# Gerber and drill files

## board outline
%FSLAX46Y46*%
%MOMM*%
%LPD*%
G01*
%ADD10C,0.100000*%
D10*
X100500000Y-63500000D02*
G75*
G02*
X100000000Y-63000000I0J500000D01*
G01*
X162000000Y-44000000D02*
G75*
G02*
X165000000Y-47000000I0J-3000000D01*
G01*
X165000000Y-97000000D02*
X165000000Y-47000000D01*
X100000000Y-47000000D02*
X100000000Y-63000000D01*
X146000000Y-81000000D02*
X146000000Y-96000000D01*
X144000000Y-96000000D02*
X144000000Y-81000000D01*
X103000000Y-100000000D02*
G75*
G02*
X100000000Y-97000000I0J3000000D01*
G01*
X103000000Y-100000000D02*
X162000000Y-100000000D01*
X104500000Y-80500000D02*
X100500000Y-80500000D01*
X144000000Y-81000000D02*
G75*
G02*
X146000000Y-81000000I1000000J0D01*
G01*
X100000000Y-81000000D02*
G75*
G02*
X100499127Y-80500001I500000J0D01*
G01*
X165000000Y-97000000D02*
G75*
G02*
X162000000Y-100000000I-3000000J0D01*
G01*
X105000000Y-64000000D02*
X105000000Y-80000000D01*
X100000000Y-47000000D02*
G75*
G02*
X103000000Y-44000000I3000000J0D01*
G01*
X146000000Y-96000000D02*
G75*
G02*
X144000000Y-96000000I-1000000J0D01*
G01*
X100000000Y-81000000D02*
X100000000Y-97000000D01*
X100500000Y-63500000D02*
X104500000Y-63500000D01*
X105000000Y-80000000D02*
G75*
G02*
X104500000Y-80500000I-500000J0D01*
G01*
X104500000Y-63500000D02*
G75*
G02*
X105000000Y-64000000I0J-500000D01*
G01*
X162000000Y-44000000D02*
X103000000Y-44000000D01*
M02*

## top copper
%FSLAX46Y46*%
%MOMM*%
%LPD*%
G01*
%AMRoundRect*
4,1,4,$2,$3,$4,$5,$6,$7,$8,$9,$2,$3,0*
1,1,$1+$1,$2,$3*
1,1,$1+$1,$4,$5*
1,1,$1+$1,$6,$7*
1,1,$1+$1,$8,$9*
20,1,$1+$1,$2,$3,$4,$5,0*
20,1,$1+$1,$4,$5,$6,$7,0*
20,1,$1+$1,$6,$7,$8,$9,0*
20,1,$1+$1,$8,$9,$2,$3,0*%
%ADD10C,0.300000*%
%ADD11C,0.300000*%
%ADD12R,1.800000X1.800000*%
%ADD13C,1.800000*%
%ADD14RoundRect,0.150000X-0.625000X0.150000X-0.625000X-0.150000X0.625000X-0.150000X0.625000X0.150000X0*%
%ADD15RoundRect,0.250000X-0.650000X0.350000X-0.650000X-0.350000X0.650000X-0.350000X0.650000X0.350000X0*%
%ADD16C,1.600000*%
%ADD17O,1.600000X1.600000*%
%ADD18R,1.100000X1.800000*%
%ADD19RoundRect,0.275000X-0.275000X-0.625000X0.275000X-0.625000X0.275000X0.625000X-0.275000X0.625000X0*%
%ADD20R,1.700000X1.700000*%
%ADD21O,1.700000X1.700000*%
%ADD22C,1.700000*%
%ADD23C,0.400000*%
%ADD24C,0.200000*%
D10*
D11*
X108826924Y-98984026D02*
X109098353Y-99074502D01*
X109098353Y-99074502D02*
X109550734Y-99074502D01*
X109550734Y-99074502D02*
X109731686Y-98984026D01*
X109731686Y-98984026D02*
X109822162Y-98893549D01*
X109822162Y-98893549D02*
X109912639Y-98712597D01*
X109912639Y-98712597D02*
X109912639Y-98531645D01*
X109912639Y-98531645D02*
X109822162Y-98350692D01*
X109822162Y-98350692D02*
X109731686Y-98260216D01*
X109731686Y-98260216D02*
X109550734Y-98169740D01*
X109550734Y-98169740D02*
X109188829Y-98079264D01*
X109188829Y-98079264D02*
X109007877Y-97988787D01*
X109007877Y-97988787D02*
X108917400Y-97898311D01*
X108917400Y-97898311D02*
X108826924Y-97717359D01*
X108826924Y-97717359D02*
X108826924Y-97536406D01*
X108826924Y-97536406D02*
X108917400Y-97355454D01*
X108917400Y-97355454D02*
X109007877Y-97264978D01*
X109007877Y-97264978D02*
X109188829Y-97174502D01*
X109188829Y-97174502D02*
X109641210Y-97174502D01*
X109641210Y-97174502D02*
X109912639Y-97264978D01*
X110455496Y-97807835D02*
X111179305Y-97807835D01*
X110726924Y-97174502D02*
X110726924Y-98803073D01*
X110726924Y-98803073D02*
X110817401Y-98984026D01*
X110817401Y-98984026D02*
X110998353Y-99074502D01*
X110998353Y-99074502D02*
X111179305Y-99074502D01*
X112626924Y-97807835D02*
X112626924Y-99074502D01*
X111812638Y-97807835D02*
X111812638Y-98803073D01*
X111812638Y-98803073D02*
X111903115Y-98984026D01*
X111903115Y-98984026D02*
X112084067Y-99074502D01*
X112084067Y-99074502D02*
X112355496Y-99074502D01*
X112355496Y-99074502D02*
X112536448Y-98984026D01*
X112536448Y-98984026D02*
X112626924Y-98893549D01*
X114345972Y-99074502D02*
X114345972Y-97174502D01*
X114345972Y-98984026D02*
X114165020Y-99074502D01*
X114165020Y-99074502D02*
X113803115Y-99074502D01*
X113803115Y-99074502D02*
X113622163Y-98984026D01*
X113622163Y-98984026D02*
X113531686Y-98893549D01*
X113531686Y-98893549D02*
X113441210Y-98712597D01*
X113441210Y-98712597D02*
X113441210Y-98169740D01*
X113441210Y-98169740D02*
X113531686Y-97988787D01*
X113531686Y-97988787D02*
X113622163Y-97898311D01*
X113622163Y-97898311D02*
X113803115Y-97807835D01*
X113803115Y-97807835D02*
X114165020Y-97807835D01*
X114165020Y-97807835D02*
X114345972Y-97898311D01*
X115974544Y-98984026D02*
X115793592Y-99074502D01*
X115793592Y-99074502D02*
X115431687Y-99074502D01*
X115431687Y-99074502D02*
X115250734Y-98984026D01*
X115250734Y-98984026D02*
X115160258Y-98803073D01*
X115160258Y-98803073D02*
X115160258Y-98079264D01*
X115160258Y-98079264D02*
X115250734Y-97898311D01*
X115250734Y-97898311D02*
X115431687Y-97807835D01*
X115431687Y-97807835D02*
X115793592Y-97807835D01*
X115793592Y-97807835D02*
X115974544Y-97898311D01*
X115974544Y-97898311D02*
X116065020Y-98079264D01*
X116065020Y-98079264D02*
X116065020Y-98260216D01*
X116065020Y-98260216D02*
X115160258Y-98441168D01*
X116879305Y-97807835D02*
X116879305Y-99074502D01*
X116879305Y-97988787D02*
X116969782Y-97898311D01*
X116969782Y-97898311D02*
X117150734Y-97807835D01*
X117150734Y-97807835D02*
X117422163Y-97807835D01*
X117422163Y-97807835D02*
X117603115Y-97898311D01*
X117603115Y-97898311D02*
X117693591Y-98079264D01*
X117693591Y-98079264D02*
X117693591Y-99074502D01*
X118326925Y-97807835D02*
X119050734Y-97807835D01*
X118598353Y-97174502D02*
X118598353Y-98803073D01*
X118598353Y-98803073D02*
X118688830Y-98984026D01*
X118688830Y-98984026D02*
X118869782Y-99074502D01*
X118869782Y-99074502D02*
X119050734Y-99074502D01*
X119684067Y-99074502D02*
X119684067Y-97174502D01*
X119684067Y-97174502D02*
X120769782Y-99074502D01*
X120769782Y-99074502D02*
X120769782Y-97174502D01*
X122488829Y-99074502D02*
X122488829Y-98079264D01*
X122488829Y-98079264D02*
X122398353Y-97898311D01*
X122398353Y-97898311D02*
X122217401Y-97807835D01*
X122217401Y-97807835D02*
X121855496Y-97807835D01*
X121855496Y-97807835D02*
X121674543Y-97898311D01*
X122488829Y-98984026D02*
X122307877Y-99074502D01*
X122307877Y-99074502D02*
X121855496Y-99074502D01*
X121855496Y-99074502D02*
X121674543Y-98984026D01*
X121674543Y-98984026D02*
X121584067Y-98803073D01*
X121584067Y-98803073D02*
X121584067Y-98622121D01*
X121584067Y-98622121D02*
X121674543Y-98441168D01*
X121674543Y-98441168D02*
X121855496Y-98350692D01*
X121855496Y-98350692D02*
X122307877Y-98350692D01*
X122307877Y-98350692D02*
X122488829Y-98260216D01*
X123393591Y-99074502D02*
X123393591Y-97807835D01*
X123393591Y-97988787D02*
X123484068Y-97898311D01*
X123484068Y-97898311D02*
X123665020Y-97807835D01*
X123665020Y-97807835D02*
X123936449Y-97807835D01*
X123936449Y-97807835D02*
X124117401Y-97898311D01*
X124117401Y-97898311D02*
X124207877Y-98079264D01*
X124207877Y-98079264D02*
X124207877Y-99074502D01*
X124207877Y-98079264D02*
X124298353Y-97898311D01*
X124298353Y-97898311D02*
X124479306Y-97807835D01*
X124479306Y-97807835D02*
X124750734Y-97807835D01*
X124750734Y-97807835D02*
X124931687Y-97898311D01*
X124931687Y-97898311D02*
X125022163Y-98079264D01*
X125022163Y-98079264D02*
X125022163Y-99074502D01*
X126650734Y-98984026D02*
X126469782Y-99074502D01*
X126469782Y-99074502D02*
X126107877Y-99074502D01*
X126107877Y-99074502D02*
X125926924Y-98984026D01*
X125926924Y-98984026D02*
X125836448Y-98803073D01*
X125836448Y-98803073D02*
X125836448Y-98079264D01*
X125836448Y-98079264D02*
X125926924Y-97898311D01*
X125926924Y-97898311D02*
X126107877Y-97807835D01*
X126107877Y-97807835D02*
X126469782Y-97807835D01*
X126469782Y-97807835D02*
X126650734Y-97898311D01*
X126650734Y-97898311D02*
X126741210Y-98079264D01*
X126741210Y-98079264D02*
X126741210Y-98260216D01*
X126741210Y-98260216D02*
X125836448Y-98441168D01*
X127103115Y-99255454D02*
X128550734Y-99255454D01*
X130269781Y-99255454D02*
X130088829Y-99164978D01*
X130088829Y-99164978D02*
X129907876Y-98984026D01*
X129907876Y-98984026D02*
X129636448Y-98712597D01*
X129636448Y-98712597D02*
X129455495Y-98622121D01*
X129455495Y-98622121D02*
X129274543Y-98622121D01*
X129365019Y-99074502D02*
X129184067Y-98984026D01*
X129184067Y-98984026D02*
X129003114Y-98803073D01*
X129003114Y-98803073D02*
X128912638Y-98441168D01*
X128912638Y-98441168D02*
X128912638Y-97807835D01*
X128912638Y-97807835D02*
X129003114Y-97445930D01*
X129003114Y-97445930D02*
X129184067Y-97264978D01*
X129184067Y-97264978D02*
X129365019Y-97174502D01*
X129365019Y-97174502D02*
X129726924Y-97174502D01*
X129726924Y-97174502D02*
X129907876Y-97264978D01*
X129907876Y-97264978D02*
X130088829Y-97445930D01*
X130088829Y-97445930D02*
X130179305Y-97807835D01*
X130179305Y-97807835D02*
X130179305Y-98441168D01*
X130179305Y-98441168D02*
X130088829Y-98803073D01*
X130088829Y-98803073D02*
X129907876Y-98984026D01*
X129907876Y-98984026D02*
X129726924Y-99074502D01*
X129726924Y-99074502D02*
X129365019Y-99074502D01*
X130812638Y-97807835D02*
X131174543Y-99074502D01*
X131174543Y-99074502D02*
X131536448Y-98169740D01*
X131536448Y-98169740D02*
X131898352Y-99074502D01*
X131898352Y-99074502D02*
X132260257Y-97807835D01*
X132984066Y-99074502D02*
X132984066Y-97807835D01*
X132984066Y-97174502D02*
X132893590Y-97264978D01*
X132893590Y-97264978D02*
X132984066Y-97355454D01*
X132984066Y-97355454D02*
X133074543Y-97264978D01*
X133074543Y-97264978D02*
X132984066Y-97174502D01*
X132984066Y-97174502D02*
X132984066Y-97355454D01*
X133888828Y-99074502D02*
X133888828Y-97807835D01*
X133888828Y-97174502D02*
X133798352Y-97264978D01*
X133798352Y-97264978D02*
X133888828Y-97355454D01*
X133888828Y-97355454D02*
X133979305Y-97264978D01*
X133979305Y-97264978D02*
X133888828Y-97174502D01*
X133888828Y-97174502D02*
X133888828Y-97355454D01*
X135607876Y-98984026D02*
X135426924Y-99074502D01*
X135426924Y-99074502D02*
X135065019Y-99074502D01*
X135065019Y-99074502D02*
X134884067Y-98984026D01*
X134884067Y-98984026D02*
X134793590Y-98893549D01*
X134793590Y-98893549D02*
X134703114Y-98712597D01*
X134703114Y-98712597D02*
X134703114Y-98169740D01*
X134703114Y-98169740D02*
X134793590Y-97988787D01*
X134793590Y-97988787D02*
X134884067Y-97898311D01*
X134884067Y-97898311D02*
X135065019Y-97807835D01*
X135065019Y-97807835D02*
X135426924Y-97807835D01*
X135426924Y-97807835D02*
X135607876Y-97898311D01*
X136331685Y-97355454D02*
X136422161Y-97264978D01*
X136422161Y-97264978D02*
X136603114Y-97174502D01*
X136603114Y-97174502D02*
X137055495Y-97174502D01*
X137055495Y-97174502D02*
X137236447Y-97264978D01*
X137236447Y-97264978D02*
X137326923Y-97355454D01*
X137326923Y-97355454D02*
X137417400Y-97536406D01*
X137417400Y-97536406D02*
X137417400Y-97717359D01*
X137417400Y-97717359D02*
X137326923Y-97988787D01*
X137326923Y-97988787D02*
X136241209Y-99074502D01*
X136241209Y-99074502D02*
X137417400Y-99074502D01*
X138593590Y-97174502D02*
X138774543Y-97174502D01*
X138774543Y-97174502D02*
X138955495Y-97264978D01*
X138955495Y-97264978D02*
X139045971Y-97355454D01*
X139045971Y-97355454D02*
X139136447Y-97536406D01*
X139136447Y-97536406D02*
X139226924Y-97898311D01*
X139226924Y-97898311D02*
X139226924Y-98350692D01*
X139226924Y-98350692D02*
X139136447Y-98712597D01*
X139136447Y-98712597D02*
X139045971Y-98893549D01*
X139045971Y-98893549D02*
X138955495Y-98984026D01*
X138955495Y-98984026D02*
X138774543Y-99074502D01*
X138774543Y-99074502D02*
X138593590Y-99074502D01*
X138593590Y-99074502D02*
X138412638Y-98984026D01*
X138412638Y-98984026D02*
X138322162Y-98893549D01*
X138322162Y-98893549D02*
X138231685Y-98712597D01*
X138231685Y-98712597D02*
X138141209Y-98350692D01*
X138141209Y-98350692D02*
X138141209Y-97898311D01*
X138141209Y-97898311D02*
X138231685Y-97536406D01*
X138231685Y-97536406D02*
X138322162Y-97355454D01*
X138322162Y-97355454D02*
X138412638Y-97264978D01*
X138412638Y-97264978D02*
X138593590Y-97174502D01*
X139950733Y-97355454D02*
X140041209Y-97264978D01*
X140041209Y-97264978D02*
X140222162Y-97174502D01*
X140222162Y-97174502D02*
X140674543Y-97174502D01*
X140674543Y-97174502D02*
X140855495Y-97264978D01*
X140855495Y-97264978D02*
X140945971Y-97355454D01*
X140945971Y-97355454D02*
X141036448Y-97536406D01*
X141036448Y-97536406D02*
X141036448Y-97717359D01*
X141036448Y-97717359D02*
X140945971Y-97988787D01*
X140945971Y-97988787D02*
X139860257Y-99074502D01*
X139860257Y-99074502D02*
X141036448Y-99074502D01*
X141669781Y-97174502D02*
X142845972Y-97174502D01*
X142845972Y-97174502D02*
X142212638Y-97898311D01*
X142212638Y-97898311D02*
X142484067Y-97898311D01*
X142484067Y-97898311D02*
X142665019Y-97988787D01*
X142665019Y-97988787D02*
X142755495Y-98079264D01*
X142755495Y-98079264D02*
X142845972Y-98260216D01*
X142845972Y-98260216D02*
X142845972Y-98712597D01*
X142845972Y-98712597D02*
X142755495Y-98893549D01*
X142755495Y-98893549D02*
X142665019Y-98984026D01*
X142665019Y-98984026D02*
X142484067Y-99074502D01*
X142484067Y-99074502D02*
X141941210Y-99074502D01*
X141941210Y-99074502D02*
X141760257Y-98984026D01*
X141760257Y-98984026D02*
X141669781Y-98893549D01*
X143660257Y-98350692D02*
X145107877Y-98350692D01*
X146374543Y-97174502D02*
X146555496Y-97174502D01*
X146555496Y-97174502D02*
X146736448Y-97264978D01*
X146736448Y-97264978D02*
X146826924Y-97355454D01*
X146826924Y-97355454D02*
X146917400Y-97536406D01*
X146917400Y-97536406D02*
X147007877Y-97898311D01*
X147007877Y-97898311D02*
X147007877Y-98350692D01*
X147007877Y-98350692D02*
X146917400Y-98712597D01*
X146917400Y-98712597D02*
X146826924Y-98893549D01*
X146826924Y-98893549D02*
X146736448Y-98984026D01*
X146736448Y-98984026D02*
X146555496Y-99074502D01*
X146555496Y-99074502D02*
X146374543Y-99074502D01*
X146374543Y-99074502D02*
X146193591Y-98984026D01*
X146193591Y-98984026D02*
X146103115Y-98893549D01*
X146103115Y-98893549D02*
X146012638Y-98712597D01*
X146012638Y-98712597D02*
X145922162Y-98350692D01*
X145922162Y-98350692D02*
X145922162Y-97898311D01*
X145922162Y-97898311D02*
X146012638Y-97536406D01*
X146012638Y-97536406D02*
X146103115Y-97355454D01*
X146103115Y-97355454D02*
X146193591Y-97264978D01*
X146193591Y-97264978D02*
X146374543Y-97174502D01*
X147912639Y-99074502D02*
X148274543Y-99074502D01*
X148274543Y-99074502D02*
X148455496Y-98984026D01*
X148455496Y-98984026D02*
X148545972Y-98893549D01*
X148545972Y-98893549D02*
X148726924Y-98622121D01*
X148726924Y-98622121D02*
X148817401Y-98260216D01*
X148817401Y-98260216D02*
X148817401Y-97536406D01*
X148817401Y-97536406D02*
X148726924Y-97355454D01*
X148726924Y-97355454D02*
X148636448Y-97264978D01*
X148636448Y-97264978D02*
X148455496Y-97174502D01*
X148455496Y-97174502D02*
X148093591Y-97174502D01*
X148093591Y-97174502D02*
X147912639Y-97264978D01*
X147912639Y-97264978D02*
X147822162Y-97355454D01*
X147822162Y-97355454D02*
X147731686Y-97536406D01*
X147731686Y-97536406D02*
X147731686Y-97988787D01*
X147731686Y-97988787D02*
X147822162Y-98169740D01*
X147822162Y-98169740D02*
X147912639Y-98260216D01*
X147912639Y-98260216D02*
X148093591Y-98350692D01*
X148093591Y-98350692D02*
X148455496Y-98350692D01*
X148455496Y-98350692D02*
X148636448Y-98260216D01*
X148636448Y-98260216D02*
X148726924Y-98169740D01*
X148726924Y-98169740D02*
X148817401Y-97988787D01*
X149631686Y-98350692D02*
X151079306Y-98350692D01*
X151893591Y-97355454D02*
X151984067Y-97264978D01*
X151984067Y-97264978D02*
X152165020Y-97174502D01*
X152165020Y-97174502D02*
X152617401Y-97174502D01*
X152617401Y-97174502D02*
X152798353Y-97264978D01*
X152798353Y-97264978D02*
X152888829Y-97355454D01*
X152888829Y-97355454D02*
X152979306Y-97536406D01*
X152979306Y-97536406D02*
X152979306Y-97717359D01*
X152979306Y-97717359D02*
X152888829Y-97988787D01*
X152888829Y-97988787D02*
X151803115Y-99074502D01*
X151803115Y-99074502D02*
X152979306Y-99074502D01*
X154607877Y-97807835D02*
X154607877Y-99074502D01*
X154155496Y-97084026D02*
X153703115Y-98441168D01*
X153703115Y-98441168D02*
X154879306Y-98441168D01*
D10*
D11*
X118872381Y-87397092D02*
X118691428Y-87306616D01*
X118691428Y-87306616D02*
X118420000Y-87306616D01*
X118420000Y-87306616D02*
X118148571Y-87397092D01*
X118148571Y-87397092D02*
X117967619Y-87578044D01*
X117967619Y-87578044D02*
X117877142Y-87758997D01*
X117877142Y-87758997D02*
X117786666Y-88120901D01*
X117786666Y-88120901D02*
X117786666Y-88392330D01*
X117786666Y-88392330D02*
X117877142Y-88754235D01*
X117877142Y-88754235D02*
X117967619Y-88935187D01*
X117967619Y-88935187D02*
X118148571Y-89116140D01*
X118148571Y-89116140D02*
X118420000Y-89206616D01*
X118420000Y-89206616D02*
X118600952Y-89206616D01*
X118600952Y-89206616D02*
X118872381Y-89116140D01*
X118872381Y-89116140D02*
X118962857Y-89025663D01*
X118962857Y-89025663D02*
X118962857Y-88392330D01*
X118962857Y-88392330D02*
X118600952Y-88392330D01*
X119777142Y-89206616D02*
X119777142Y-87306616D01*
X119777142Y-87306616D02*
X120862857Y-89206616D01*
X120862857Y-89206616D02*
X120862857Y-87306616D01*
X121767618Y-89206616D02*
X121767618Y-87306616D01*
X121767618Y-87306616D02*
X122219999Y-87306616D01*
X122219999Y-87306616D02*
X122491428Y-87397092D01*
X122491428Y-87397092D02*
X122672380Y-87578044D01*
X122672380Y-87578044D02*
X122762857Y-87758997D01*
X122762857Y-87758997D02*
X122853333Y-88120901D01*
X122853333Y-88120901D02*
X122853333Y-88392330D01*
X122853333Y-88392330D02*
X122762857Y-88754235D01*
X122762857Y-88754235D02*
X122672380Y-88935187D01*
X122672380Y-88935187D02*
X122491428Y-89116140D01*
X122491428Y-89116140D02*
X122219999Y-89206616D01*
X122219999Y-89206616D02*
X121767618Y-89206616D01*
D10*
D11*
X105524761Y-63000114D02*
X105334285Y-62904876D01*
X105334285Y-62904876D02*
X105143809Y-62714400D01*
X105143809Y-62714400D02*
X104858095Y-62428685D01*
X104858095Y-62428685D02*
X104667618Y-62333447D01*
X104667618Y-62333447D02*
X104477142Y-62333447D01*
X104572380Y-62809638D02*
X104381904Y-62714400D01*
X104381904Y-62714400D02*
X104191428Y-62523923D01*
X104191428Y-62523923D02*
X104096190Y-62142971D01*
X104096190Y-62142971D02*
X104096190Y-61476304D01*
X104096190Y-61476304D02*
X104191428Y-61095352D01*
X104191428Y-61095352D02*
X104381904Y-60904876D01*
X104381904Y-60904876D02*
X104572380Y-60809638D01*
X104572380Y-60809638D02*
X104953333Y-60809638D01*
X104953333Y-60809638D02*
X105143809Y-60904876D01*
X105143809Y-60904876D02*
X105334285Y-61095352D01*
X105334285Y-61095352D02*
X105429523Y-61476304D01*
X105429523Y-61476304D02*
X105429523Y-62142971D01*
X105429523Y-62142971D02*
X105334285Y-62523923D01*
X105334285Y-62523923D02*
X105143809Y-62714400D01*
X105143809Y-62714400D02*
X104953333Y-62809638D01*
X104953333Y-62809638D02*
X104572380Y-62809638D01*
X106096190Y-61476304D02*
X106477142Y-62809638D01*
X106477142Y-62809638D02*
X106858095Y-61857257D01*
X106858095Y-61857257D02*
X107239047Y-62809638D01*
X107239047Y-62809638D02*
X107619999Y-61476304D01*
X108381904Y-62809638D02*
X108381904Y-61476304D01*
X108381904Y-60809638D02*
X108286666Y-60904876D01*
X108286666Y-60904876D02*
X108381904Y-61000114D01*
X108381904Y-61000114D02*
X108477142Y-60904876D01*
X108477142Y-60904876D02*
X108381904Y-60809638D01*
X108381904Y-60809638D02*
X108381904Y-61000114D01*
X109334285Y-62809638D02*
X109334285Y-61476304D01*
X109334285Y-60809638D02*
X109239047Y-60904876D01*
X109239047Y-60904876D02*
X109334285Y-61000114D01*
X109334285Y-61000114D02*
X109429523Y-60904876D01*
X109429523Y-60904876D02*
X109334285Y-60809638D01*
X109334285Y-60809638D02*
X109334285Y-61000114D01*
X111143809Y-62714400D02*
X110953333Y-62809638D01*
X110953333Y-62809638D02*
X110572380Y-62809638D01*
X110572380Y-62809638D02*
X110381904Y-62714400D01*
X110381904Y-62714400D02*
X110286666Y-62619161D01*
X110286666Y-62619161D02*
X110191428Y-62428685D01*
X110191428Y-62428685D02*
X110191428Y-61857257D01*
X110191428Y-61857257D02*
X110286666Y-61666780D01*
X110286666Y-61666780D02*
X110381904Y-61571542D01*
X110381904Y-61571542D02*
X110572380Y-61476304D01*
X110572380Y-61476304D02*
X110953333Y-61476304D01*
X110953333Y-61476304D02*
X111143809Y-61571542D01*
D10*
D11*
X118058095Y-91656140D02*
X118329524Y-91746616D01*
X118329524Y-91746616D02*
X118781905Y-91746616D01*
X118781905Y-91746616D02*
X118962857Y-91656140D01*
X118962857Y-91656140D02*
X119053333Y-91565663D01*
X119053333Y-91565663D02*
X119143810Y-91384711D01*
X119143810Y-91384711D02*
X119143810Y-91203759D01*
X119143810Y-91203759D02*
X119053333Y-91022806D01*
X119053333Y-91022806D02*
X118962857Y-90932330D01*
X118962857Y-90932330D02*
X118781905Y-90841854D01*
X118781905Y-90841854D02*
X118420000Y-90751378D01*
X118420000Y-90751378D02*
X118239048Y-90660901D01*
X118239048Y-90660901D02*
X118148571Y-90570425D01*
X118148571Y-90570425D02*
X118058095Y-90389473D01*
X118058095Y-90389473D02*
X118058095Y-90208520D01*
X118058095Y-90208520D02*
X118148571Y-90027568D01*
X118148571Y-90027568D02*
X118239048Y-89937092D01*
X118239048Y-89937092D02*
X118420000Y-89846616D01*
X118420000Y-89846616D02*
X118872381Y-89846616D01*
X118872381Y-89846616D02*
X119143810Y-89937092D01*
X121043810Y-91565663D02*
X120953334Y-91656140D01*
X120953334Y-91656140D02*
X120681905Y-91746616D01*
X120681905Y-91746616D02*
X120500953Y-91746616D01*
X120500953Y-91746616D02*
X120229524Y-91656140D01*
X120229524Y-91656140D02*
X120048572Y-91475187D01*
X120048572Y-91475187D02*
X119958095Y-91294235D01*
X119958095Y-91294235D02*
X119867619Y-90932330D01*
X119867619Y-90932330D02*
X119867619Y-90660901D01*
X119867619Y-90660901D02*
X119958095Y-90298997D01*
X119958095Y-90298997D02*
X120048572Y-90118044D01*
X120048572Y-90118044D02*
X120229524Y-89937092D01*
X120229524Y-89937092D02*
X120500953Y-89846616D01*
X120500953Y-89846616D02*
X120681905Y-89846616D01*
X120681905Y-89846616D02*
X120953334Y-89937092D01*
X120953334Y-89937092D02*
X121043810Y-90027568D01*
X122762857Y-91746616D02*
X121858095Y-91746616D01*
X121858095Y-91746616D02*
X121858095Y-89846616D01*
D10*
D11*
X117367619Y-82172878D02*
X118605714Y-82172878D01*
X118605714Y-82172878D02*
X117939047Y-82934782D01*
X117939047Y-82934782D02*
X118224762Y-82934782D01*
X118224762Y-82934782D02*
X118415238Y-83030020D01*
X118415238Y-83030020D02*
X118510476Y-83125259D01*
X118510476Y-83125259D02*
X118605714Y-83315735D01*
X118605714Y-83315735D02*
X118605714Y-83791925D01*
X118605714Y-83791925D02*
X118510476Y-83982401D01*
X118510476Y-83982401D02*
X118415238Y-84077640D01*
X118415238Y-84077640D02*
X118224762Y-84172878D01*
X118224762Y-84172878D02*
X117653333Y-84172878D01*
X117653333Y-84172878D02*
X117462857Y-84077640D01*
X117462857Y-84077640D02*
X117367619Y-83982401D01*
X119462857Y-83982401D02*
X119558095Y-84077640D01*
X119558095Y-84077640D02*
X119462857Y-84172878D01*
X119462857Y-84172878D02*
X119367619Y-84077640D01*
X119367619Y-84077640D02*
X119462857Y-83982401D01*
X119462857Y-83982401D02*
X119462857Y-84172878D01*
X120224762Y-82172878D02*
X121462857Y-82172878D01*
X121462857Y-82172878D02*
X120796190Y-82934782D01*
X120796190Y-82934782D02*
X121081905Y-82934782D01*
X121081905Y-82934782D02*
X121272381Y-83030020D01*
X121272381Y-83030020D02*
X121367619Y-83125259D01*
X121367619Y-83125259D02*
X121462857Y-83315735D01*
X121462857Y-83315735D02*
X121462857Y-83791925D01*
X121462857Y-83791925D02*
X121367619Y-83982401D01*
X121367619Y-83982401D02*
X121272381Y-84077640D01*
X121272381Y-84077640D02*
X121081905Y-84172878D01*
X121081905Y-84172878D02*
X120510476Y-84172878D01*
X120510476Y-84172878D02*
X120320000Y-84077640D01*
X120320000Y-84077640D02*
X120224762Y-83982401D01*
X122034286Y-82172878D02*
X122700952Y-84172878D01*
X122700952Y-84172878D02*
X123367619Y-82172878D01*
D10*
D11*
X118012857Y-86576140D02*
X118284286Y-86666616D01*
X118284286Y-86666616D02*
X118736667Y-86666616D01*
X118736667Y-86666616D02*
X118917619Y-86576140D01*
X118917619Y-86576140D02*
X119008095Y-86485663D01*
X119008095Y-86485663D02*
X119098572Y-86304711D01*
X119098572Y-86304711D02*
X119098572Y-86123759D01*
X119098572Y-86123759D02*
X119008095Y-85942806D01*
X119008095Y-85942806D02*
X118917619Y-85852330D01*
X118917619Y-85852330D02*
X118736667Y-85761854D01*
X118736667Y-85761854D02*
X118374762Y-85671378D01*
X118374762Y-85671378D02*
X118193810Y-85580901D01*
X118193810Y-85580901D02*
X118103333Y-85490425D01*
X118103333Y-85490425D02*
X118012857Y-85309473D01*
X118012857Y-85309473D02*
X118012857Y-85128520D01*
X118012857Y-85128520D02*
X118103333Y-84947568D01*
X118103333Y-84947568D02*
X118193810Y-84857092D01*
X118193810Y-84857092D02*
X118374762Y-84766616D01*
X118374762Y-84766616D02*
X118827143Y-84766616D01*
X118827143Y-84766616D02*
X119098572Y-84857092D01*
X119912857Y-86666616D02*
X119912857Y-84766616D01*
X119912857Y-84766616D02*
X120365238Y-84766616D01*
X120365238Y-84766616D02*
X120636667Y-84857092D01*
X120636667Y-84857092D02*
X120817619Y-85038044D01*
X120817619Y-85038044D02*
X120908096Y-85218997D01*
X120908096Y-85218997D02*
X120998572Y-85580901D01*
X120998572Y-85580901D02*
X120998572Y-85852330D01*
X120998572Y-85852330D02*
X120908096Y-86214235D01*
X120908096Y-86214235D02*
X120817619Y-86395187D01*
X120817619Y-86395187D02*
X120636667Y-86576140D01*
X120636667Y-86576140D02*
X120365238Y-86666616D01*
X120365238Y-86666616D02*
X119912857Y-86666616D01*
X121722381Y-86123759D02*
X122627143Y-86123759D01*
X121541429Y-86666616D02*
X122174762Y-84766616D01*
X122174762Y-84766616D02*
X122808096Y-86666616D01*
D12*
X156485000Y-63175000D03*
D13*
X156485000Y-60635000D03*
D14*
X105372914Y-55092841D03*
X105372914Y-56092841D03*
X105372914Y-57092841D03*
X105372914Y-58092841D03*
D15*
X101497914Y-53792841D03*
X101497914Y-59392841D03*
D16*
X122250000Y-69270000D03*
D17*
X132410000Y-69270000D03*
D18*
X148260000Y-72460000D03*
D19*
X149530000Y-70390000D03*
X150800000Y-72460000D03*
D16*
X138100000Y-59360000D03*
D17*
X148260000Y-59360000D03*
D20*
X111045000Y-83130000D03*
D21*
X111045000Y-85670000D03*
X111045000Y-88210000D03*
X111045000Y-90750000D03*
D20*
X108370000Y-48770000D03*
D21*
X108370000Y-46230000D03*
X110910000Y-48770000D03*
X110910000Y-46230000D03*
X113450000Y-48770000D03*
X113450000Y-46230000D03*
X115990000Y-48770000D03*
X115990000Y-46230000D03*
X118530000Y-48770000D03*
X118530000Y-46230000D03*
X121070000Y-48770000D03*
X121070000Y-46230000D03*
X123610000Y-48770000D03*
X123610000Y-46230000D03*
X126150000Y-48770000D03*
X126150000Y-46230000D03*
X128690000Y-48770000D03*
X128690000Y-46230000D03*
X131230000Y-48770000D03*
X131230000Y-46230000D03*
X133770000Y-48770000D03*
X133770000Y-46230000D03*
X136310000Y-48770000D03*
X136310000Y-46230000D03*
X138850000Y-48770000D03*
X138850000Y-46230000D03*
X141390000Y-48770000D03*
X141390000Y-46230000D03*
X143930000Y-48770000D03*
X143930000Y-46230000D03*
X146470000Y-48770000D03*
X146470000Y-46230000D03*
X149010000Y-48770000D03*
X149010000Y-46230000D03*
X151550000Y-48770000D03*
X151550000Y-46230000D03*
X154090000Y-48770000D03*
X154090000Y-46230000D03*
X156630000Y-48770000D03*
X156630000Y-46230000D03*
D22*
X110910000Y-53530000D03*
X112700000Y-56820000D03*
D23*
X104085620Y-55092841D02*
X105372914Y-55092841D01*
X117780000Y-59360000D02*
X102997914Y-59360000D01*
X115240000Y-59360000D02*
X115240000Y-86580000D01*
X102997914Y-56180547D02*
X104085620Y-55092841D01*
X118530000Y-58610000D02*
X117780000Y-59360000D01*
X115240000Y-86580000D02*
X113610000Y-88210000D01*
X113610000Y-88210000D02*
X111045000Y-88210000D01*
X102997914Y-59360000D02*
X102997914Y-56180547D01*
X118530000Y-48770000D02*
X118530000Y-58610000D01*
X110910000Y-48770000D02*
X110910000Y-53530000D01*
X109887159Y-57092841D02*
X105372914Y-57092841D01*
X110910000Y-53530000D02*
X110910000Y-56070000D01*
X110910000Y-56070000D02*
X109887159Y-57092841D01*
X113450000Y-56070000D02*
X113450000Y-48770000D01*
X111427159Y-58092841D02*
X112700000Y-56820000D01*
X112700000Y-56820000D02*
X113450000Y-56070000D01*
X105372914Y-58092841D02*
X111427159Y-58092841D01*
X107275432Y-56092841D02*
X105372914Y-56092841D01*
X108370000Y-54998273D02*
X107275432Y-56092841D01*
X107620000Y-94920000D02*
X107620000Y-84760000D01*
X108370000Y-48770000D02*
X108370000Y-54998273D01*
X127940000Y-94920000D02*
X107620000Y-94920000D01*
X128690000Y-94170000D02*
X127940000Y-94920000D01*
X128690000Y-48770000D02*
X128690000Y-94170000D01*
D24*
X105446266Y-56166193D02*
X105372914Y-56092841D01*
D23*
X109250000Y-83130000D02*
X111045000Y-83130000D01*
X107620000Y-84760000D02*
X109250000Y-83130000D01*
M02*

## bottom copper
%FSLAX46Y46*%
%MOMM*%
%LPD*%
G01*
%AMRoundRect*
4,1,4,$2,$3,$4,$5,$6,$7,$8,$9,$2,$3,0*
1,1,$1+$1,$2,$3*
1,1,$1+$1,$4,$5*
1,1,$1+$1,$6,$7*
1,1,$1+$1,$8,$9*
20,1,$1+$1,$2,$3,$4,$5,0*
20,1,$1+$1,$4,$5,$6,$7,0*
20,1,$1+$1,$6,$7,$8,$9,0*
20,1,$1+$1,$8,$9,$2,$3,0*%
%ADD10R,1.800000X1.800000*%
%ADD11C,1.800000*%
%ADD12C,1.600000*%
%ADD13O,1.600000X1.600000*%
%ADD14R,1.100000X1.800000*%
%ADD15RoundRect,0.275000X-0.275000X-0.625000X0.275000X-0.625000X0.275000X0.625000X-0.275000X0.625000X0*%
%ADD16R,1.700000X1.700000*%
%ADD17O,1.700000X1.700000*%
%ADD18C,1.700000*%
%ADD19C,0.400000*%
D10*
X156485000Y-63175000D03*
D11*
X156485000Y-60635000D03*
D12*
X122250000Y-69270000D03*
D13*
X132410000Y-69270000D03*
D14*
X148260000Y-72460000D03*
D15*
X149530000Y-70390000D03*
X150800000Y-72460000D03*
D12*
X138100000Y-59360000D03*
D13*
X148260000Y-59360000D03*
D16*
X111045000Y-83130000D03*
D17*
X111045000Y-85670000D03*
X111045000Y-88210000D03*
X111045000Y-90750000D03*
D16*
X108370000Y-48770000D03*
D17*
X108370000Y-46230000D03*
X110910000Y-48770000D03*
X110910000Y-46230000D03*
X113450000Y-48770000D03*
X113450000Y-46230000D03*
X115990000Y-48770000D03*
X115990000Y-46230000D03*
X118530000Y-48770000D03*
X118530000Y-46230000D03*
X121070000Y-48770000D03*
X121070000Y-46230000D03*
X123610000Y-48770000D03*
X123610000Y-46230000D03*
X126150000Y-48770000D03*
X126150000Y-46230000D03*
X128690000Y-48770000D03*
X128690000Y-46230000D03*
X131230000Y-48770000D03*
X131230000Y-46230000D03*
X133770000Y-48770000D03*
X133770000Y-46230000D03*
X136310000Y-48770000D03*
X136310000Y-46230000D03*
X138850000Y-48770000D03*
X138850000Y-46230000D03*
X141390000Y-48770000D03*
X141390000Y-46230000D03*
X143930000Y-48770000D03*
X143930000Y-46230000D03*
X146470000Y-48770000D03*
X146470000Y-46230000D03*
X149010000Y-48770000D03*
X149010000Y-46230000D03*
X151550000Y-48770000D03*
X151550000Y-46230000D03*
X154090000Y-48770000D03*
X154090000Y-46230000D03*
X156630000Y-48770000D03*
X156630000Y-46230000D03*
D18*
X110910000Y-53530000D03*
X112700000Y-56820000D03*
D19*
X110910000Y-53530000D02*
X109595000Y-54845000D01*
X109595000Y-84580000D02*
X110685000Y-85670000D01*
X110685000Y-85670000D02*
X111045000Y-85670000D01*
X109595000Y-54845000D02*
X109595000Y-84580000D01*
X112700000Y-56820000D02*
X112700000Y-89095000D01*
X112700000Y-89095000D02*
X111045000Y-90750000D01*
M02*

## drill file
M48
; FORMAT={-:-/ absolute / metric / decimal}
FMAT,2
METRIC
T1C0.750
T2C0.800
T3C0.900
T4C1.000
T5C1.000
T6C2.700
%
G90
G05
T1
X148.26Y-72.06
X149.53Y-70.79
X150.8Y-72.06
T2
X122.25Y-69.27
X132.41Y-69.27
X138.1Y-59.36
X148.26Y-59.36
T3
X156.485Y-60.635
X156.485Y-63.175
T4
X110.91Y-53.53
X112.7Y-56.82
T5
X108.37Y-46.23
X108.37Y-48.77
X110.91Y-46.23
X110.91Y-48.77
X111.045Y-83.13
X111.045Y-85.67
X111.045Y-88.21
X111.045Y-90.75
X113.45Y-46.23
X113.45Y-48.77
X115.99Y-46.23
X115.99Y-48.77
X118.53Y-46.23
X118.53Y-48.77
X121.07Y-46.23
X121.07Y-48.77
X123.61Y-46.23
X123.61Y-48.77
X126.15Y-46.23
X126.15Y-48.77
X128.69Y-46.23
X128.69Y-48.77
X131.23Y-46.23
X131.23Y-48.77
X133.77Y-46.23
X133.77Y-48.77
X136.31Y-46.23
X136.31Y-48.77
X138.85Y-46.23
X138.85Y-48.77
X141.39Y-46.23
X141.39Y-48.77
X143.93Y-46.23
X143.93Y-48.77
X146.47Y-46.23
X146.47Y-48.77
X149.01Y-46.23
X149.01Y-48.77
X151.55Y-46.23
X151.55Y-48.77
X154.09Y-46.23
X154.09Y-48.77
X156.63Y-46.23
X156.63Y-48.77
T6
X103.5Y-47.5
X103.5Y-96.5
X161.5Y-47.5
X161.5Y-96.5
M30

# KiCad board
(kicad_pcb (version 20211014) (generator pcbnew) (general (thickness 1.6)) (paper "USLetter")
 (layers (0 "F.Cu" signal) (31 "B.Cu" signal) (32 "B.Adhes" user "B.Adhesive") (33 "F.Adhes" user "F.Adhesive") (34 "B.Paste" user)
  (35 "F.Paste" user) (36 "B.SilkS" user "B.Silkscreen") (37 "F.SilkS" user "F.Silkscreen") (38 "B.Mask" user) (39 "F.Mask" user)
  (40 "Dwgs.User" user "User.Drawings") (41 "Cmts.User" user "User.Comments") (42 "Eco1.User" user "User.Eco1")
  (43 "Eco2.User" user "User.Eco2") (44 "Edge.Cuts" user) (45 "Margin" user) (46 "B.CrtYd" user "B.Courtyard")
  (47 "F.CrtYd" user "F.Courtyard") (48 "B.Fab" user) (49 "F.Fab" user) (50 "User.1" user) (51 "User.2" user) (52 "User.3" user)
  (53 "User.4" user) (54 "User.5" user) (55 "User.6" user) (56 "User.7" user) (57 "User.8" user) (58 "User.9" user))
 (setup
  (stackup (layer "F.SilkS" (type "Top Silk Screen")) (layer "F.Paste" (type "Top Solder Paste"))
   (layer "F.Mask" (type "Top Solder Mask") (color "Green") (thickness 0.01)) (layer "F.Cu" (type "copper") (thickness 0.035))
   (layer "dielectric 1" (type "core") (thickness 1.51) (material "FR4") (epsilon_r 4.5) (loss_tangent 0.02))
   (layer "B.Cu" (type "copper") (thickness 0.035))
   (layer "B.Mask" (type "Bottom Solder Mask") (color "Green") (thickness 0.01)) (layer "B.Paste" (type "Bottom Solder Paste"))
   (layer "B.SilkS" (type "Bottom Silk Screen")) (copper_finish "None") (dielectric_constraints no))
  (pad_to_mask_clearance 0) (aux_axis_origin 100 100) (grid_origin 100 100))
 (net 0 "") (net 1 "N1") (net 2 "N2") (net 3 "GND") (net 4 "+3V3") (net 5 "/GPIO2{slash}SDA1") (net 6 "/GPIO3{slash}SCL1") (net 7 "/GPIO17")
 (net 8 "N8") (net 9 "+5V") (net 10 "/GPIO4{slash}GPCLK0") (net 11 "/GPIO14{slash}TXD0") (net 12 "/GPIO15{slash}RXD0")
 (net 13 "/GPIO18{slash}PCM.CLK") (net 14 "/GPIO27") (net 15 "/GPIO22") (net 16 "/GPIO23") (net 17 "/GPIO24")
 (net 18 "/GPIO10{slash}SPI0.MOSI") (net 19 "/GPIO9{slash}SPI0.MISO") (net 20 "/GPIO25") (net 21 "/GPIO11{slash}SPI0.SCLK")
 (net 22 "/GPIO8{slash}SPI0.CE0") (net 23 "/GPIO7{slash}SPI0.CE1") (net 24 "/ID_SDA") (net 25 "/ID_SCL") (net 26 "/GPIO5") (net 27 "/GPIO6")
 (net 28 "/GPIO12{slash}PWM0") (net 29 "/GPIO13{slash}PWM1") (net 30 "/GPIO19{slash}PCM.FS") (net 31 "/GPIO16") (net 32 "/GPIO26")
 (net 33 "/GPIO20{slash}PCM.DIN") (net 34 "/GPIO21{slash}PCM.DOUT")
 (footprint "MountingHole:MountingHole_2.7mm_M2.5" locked (layer "F.Cu") (at 161.5 47.5)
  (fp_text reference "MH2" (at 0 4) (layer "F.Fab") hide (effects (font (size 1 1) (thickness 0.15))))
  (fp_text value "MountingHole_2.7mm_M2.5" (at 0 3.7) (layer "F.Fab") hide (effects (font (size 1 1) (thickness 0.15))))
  (pad "" np_thru_hole circle locked (at 0 0) (size 2.7 2.7) (drill 2.7) (layers *.Cu *.Mask)))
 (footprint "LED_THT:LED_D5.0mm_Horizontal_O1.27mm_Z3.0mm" (layer "F.Cu") (at 156.485 63.175 90)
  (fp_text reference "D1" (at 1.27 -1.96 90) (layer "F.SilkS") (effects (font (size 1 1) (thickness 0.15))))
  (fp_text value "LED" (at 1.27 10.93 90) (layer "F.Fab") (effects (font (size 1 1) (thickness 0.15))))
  (pad "1" thru_hole rect (at 0 0 90) (size 1.8 1.8) (drill 0.9) (layers *.Cu *.Mask) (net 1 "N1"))
  (pad "2" thru_hole circle (at 2.54 0 90) (size 1.8 1.8) (drill 0.9) (layers *.Cu *.Mask) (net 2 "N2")))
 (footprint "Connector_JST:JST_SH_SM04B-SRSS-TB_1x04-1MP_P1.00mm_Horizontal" (layer "F.Cu") (at 103.372914 56.592841 -90)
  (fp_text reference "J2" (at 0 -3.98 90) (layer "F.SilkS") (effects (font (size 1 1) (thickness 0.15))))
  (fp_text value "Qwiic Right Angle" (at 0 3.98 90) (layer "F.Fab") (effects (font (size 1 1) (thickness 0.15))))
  (pad "1" smd roundrect (at -1.5 -2 270) (size 0.6 1.55) (layers "F.Cu" "F.Paste" "F.Mask") (roundrect_rratio 0.25) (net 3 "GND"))
  (pad "2" smd roundrect (at -0.5 -2 270) (size 0.6 1.55) (layers "F.Cu" "F.Paste" "F.Mask") (roundrect_rratio 0.25) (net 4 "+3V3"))
  (pad "3" smd roundrect (at 0.5 -2 270) (size 0.6 1.55) (layers "F.Cu" "F.Paste" "F.Mask") (roundrect_rratio 0.25)
   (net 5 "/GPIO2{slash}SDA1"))
  (pad "4" smd roundrect (at 1.5 -2 270) (size 0.6 1.55) (layers "F.Cu" "F.Paste" "F.Mask") (roundrect_rratio 0.25)
   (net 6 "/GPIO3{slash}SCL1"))
  (pad "MP" smd roundrect (at -2.8 1.875 270) (size 1.2 1.8) (layers "F.Cu" "F.Paste" "F.Mask") (roundrect_rratio 0.2083333333))
  (pad "MP" smd roundrect (at 2.8 1.875 270) (size 1.2 1.8) (layers "F.Cu" "F.Paste" "F.Mask") (roundrect_rratio 0.2083333333)))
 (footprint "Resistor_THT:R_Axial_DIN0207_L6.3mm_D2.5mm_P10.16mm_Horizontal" (layer "F.Cu") (at 122.25 69.27)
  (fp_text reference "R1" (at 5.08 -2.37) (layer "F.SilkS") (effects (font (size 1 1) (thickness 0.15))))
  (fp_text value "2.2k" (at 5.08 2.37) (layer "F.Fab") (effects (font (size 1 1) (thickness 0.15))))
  (pad "1" thru_hole circle (at 0 0) (size 1.6 1.6) (drill 0.8) (layers *.Cu *.Mask) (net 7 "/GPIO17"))
  (pad "2" thru_hole oval (at 10.16 0) (size 1.6 1.6) (drill 0.8) (layers *.Cu *.Mask) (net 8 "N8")))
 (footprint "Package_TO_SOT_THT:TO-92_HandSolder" (layer "F.Cu") (at 148.26 72.06)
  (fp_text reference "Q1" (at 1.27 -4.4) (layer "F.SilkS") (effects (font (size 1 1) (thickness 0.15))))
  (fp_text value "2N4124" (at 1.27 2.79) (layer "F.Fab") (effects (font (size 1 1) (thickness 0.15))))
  (pad "1" thru_hole rect (at 0 0) (size 1.1 1.8) (drill 0.75 (offset 0 0.4)) (layers *.Cu *.Mask) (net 3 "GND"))
  (pad "2" thru_hole roundrect (at 1.27 -1.27) (size 1.1 1.8) (drill 0.75 (offset 0 -0.4)) (layers *.Cu *.Mask) (roundrect_rratio 0.25)
   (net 8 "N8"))
  (pad "3" thru_hole roundrect (at 2.54 0) (size 1.1 1.8) (drill 0.75 (offset 0 0.4)) (layers *.Cu *.Mask) (roundrect_rratio 0.25)
   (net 1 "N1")))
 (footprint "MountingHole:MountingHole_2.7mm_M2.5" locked (layer "F.Cu") (at 103.5 96.5)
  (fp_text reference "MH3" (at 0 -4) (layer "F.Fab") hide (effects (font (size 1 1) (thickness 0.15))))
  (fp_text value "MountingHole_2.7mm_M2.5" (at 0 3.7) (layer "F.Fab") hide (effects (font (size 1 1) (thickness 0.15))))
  (pad "" np_thru_hole circle locked (at 0 0) (size 2.7 2.7) (drill 2.7) (layers *.Cu *.Mask)))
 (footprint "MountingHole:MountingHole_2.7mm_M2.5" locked (layer "F.Cu") (at 103.5 47.5)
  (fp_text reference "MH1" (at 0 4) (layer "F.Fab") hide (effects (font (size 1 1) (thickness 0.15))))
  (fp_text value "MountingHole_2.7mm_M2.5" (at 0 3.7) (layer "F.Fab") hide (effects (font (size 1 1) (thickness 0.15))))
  (pad "" np_thru_hole circle locked (at 0 0) (size 2.7 2.7) (drill 2.7) (layers *.Cu *.Mask)))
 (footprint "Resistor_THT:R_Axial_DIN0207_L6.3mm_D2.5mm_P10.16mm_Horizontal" (layer "F.Cu") (at 138.1 59.36)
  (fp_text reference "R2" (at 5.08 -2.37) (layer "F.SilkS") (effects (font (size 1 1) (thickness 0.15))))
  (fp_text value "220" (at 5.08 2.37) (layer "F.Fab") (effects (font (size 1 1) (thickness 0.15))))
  (pad "1" thru_hole circle (at 0 0) (size 1.6 1.6) (drill 0.8) (layers *.Cu *.Mask) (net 4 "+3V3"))
  (pad "2" thru_hole oval (at 10.16 0) (size 1.6 1.6) (drill 0.8) (layers *.Cu *.Mask) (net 2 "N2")))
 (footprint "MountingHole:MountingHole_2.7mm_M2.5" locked (layer "F.Cu") (at 161.5 96.5)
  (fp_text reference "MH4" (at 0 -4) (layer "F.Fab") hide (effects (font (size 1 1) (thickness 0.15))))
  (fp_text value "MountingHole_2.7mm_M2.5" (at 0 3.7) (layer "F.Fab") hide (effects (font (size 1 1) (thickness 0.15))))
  (pad "" np_thru_hole circle locked (at 0 0) (size 2.7 2.7) (drill 2.7) (layers *.Cu *.Mask)))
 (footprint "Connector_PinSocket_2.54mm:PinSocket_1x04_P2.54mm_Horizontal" (layer "F.Cu") (at 111.045 83.13)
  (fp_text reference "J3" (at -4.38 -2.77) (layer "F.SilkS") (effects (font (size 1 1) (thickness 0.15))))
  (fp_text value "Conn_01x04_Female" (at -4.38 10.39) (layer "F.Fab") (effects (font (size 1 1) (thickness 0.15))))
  (pad "1" thru_hole rect (at 0 0) (size 1.7 1.7) (drill 1) (layers *.Cu *.Mask) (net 4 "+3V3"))
  (pad "2" thru_hole oval (at 0 2.54) (size 1.7 1.7) (drill 1) (layers *.Cu *.Mask) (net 5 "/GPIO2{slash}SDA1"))
  (pad "3" thru_hole oval (at 0 5.08) (size 1.7 1.7) (drill 1) (layers *.Cu *.Mask) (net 3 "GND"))
  (pad "4" thru_hole oval (at 0 7.62) (size 1.7 1.7) (drill 1) (layers *.Cu *.Mask) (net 6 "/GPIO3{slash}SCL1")))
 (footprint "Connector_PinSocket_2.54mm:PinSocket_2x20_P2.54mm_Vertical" (layer "B.Cu") (at 108.37 48.77 -90)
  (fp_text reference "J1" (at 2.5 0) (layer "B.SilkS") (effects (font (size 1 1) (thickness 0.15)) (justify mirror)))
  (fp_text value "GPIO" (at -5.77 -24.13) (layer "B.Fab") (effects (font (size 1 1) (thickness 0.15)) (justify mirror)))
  (pad "1" thru_hole rect locked (at 0 0 270) (size 1.7 1.7) (drill 1) (layers *.Cu *.Mask) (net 4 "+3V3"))
  (pad "2" thru_hole oval locked (at -2.54 0 270) (size 1.7 1.7) (drill 1) (layers *.Cu *.Mask) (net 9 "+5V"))
  (pad "3" thru_hole oval locked (at 0 -2.54 270) (size 1.7 1.7) (drill 1) (layers *.Cu *.Mask) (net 5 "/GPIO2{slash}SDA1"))
  (pad "4" thru_hole oval locked (at -2.54 -2.54 270) (size 1.7 1.7) (drill 1) (layers *.Cu *.Mask) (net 9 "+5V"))
  (pad "5" thru_hole oval locked (at 0 -5.08 270) (size 1.7 1.7) (drill 1) (layers *.Cu *.Mask) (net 6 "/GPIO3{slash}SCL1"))
  (pad "6" thru_hole oval locked (at -2.54 -5.08 270) (size 1.7 1.7) (drill 1) (layers *.Cu *.Mask) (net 3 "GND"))
  (pad "7" thru_hole oval locked (at 0 -7.62 270) (size 1.7 1.7) (drill 1) (layers *.Cu *.Mask) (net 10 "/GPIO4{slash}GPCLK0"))
  (pad "8" thru_hole oval locked (at -2.54 -7.62 270) (size 1.7 1.7) (drill 1) (layers *.Cu *.Mask) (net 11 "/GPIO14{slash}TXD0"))
  (pad "9" thru_hole oval locked (at 0 -10.16 270) (size 1.7 1.7) (drill 1) (layers *.Cu *.Mask) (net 3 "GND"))
  (pad "10" thru_hole oval locked (at -2.54 -10.16 270) (size 1.7 1.7) (drill 1) (layers *.Cu *.Mask) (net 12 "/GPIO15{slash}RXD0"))
  (pad "11" thru_hole oval locked (at 0 -12.7 270) (size 1.7 1.7) (drill 1) (layers *.Cu *.Mask) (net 7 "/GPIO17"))
  (pad "12" thru_hole oval locked (at -2.54 -12.7 270) (size 1.7 1.7) (drill 1) (layers *.Cu *.Mask) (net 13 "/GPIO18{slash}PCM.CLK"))
  (pad "13" thru_hole oval locked (at 0 -15.24 270) (size 1.7 1.7) (drill 1) (layers *.Cu *.Mask) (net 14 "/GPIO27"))
  (pad "14" thru_hole oval locked (at -2.54 -15.24 270) (size 1.7 1.7) (drill 1) (layers *.Cu *.Mask) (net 3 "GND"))
  (pad "15" thru_hole oval locked (at 0 -17.78 270) (size 1.7 1.7) (drill 1) (layers *.Cu *.Mask) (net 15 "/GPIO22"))
  (pad "16" thru_hole oval locked (at -2.54 -17.78 270) (size 1.7 1.7) (drill 1) (layers *.Cu *.Mask) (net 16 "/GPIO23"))
  (pad "17" thru_hole oval locked (at 0 -20.32 270) (size 1.7 1.7) (drill 1) (layers *.Cu *.Mask) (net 4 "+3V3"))
  (pad "18" thru_hole oval locked (at -2.54 -20.32 270) (size 1.7 1.7) (drill 1) (layers *.Cu *.Mask) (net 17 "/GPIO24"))
  (pad "19" thru_hole oval locked (at 0 -22.86 270) (size 1.7 1.7) (drill 1) (layers *.Cu *.Mask) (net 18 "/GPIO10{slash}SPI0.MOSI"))
  (pad "20" thru_hole oval locked (at -2.54 -22.86 270) (size 1.7 1.7) (drill 1) (layers *.Cu *.Mask) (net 3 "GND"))
  (pad "21" thru_hole oval locked (at 0 -25.4 270) (size 1.7 1.7) (drill 1) (layers *.Cu *.Mask) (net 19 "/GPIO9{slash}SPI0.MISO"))
  (pad "22" thru_hole oval locked (at -2.54 -25.4 270) (size 1.7 1.7) (drill 1) (layers *.Cu *.Mask) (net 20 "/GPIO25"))
  (pad "23" thru_hole oval locked (at 0 -27.94 270) (size 1.7 1.7) (drill 1) (layers *.Cu *.Mask) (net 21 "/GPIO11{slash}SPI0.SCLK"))
  (pad "24" thru_hole oval locked (at -2.54 -27.94 270) (size 1.7 1.7) (drill 1) (layers *.Cu *.Mask) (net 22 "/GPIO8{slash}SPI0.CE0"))
  (pad "25" thru_hole oval locked (at 0 -30.48 270) (size 1.7 1.7) (drill 1) (layers *.Cu *.Mask) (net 3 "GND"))
  (pad "26" thru_hole oval locked (at -2.54 -30.48 270) (size 1.7 1.7) (drill 1) (layers *.Cu *.Mask) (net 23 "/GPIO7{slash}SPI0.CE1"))
  (pad "27" thru_hole oval locked (at 0 -33.02 270) (size 1.7 1.7) (drill 1) (layers *.Cu *.Mask) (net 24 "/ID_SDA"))
  (pad "28" thru_hole oval locked (at -2.54 -33.02 270) (size 1.7 1.7) (drill 1) (layers *.Cu *.Mask) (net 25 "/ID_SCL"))
  (pad "29" thru_hole oval locked (at 0 -35.56 270) (size 1.7 1.7) (drill 1) (layers *.Cu *.Mask) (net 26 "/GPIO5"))
  (pad "30" thru_hole oval locked (at -2.54 -35.56 270) (size 1.7 1.7) (drill 1) (layers *.Cu *.Mask) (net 3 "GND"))
  (pad "31" thru_hole oval locked (at 0 -38.1 270) (size 1.7 1.7) (drill 1) (layers *.Cu *.Mask) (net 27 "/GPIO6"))
  (pad "32" thru_hole oval locked (at -2.54 -38.1 270) (size 1.7 1.7) (drill 1) (layers *.Cu *.Mask) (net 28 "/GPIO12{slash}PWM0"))
  (pad "33" thru_hole oval locked (at 0 -40.64 270) (size 1.7 1.7) (drill 1) (layers *.Cu *.Mask) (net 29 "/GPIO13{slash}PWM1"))
  (pad "34" thru_hole oval locked (at -2.54 -40.64 270) (size 1.7 1.7) (drill 1) (layers *.Cu *.Mask) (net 3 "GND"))
  (pad "35" thru_hole oval locked (at 0 -43.18 270) (size 1.7 1.7) (drill 1) (layers *.Cu *.Mask) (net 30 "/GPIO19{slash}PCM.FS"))
  (pad "36" thru_hole oval locked (at -2.54 -43.18 270) (size 1.7 1.7) (drill 1) (layers *.Cu *.Mask) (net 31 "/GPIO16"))
  (pad "37" thru_hole oval locked (at 0 -45.72 270) (size 1.7 1.7) (drill 1) (layers *.Cu *.Mask) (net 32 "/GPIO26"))
  (pad "38" thru_hole oval locked (at -2.54 -45.72 270) (size 1.7 1.7) (drill 1) (layers *.Cu *.Mask) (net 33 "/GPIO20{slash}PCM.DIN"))
  (pad "39" thru_hole oval locked (at 0 -48.26 270) (size 1.7 1.7) (drill 1) (layers *.Cu *.Mask) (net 3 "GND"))
  (pad "40" thru_hole oval locked (at -2.54 -48.26 270) (size 1.7 1.7) (drill 1) (layers *.Cu *.Mask) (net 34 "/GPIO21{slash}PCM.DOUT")))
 (gr_arc (start 100.5 63.5) (mid 100.146447 63.353553) (end 100 63) (layer "Edge.Cuts") (width 0.1))
 (gr_arc (start 162 44) (mid 164.12132 44.87868) (end 165 47) (layer "Edge.Cuts") (width 0.1))
 (gr_line (start 165 97) (end 165 47) (layer "Edge.Cuts") (width 0.1))
 (gr_line (start 100 47) (end 100 63) (layer "Edge.Cuts") (width 0.1))
 (gr_line (start 146 81) (end 146 96) (layer "Edge.Cuts") (width 0.1))
 (gr_line (start 144 96) (end 144 81) (layer "Edge.Cuts") (width 0.1))
 (gr_arc (start 103 100) (mid 100.87868 99.12132) (end 100 97) (layer "Edge.Cuts") (width 0.1))
 (gr_line (start 103 100) (end 162 100) (layer "Edge.Cuts") (width 0.1))
 (gr_line (start 104.5 80.5) (end 100.5 80.5) (layer "Edge.Cuts") (width 0.1))
 (gr_arc (start 144 81) (mid 145 80) (end 146 81) (layer "Edge.Cuts") (width 0.1))
 (gr_arc (start 100 81) (mid 100.146138 80.646755) (end 100.499127 80.500001) (layer "Edge.Cuts") (width 0.1))
 (gr_arc (start 165 97) (mid 164.12132 99.12132) (end 162 100) (layer "Edge.Cuts") (width 0.1))
 (gr_line (start 105 64) (end 105 80) (layer "Edge.Cuts") (width 0.1))
 (gr_arc (start 100 47) (mid 100.87868 44.87868) (end 103 44) (layer "Edge.Cuts") (width 0.1))
 (gr_arc (start 146 96) (mid 145 97) (end 144 96) (layer "Edge.Cuts") (width 0.1))
 (gr_line (start 100 81) (end 100 97) (layer "Edge.Cuts") (width 0.1))
 (gr_line (start 100.5 63.5) (end 104.5 63.5) (layer "Edge.Cuts") (width 0.1))
 (gr_arc (start 105 80) (mid 104.853553 80.353553) (end 104.5 80.5) (layer "Edge.Cuts") (width 0.1))
 (gr_arc (start 104.5 63.5) (mid 104.853553 63.646447) (end 105 64) (layer "Edge.Cuts") (width 0.1))
 (gr_line (start 162 44) (end 103 44) (layer "Edge.Cuts") (width 0.1))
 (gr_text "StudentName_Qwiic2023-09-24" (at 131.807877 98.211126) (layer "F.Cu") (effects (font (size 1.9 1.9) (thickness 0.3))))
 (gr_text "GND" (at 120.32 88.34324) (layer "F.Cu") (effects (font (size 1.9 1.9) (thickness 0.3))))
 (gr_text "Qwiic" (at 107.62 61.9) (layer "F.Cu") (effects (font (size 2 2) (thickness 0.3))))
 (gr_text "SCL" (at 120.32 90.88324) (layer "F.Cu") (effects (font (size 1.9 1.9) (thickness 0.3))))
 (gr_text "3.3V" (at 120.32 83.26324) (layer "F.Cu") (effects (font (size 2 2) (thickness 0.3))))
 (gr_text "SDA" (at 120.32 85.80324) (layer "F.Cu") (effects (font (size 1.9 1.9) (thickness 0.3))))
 (segment (start 104.08562 55.092841) (end 105.372914 55.092841) (width 0.4) (layer "F.Cu") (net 3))
 (segment (start 117.78 59.36) (end 102.997914 59.36) (width 0.4) (layer "F.Cu") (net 3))
 (segment (start 115.24 59.36) (end 115.24 86.58) (width 0.4) (layer "F.Cu") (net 3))
 (segment (start 102.997914 56.180547) (end 104.08562 55.092841) (width 0.4) (layer "F.Cu") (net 3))
 (segment (start 118.53 58.61) (end 117.78 59.36) (width 0.4) (layer "F.Cu") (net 3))
 (segment (start 115.24 86.58) (end 113.61 88.21) (width 0.4) (layer "F.Cu") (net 3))
 (segment (start 113.61 88.21) (end 111.045 88.21) (width 0.4) (layer "F.Cu") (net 3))
 (segment (start 102.997914 59.36) (end 102.997914 56.180547) (width 0.4) (layer "F.Cu") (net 3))
 (segment (start 118.53 48.77) (end 118.53 58.61) (width 0.4) (layer "F.Cu") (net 3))
 (segment (start 110.91 48.77) (end 110.91 53.53) (width 0.4) (layer "F.Cu") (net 5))
 (segment (start 109.887159 57.092841) (end 105.372914 57.092841) (width 0.4) (layer "F.Cu") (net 5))
 (segment (start 110.91 53.53) (end 110.91 56.07) (width 0.4) (layer "F.Cu") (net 5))
 (segment (start 110.91 56.07) (end 109.887159 57.092841) (width 0.4) (layer "F.Cu") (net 5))
 (via (at 110.91 53.53) (size 1.7) (drill 1) (layers "F.Cu" "B.Cu") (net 5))
 (segment (start 110.91 53.53) (end 109.595 54.845) (width 0.4) (layer "B.Cu") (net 5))
 (segment (start 109.595 84.58) (end 110.685 85.67) (width 0.4) (layer "B.Cu") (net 5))
 (segment (start 110.685 85.67) (end 111.045 85.67) (width 0.4) (layer "B.Cu") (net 5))
 (segment (start 109.595 54.845) (end 109.595 84.58) (width 0.4) (layer "B.Cu") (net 5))
 (segment (start 113.45 56.07) (end 113.45 48.77) (width 0.4) (layer "F.Cu") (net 6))
 (segment (start 111.427159 58.092841) (end 112.7 56.82) (width 0.4) (layer "F.Cu") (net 6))
 (segment (start 112.7 56.82) (end 113.45 56.07) (width 0.4) (layer "F.Cu") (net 6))
 (segment (start 105.372914 58.092841) (end 111.427159 58.092841) (width 0.4) (layer "F.Cu") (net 6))
 (via (at 112.7 56.82) (size 1.7) (drill 1) (layers "F.Cu" "B.Cu") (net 6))
 (segment (start 112.7 56.82) (end 112.7 89.095) (width 0.4) (layer "B.Cu") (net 6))
 (segment (start 112.7 89.095) (end 111.045 90.75) (width 0.4) (layer "B.Cu") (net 6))
 (segment (start 107.275432 56.092841) (end 105.372914 56.092841) (width 0.4) (layer "F.Cu") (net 4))
 (segment (start 108.37 54.998273) (end 107.275432 56.092841) (width 0.4) (layer "F.Cu") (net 4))
 (segment (start 107.62 94.92) (end 107.62 84.76) (width 0.4) (layer "F.Cu") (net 4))
 (segment (start 108.37 48.77) (end 108.37 54.998273) (width 0.4) (layer "F.Cu") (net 4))
 (segment (start 127.94 94.92) (end 107.62 94.92) (width 0.4) (layer "F.Cu") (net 4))
 (segment (start 128.69 94.17) (end 127.94 94.92) (width 0.4) (layer "F.Cu") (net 4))
 (segment (start 128.69 48.77) (end 128.69 94.17) (width 0.4) (layer "F.Cu") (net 4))
 (segment (start 105.446266 56.166193) (end 105.372914 56.092841) (width 0.2) (layer "F.Cu") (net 4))
 (segment (start 109.25 83.13) (end 111.045 83.13) (width 0.4) (layer "F.Cu") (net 4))
 (segment (start 107.62 84.76) (end 109.25 83.13) (width 0.4) (layer "F.Cu") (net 4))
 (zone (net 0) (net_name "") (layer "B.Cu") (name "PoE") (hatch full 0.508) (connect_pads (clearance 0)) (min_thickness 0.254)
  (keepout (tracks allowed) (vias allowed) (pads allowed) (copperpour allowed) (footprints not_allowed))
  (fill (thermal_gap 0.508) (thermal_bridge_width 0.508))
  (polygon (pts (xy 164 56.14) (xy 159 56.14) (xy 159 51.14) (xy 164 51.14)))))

